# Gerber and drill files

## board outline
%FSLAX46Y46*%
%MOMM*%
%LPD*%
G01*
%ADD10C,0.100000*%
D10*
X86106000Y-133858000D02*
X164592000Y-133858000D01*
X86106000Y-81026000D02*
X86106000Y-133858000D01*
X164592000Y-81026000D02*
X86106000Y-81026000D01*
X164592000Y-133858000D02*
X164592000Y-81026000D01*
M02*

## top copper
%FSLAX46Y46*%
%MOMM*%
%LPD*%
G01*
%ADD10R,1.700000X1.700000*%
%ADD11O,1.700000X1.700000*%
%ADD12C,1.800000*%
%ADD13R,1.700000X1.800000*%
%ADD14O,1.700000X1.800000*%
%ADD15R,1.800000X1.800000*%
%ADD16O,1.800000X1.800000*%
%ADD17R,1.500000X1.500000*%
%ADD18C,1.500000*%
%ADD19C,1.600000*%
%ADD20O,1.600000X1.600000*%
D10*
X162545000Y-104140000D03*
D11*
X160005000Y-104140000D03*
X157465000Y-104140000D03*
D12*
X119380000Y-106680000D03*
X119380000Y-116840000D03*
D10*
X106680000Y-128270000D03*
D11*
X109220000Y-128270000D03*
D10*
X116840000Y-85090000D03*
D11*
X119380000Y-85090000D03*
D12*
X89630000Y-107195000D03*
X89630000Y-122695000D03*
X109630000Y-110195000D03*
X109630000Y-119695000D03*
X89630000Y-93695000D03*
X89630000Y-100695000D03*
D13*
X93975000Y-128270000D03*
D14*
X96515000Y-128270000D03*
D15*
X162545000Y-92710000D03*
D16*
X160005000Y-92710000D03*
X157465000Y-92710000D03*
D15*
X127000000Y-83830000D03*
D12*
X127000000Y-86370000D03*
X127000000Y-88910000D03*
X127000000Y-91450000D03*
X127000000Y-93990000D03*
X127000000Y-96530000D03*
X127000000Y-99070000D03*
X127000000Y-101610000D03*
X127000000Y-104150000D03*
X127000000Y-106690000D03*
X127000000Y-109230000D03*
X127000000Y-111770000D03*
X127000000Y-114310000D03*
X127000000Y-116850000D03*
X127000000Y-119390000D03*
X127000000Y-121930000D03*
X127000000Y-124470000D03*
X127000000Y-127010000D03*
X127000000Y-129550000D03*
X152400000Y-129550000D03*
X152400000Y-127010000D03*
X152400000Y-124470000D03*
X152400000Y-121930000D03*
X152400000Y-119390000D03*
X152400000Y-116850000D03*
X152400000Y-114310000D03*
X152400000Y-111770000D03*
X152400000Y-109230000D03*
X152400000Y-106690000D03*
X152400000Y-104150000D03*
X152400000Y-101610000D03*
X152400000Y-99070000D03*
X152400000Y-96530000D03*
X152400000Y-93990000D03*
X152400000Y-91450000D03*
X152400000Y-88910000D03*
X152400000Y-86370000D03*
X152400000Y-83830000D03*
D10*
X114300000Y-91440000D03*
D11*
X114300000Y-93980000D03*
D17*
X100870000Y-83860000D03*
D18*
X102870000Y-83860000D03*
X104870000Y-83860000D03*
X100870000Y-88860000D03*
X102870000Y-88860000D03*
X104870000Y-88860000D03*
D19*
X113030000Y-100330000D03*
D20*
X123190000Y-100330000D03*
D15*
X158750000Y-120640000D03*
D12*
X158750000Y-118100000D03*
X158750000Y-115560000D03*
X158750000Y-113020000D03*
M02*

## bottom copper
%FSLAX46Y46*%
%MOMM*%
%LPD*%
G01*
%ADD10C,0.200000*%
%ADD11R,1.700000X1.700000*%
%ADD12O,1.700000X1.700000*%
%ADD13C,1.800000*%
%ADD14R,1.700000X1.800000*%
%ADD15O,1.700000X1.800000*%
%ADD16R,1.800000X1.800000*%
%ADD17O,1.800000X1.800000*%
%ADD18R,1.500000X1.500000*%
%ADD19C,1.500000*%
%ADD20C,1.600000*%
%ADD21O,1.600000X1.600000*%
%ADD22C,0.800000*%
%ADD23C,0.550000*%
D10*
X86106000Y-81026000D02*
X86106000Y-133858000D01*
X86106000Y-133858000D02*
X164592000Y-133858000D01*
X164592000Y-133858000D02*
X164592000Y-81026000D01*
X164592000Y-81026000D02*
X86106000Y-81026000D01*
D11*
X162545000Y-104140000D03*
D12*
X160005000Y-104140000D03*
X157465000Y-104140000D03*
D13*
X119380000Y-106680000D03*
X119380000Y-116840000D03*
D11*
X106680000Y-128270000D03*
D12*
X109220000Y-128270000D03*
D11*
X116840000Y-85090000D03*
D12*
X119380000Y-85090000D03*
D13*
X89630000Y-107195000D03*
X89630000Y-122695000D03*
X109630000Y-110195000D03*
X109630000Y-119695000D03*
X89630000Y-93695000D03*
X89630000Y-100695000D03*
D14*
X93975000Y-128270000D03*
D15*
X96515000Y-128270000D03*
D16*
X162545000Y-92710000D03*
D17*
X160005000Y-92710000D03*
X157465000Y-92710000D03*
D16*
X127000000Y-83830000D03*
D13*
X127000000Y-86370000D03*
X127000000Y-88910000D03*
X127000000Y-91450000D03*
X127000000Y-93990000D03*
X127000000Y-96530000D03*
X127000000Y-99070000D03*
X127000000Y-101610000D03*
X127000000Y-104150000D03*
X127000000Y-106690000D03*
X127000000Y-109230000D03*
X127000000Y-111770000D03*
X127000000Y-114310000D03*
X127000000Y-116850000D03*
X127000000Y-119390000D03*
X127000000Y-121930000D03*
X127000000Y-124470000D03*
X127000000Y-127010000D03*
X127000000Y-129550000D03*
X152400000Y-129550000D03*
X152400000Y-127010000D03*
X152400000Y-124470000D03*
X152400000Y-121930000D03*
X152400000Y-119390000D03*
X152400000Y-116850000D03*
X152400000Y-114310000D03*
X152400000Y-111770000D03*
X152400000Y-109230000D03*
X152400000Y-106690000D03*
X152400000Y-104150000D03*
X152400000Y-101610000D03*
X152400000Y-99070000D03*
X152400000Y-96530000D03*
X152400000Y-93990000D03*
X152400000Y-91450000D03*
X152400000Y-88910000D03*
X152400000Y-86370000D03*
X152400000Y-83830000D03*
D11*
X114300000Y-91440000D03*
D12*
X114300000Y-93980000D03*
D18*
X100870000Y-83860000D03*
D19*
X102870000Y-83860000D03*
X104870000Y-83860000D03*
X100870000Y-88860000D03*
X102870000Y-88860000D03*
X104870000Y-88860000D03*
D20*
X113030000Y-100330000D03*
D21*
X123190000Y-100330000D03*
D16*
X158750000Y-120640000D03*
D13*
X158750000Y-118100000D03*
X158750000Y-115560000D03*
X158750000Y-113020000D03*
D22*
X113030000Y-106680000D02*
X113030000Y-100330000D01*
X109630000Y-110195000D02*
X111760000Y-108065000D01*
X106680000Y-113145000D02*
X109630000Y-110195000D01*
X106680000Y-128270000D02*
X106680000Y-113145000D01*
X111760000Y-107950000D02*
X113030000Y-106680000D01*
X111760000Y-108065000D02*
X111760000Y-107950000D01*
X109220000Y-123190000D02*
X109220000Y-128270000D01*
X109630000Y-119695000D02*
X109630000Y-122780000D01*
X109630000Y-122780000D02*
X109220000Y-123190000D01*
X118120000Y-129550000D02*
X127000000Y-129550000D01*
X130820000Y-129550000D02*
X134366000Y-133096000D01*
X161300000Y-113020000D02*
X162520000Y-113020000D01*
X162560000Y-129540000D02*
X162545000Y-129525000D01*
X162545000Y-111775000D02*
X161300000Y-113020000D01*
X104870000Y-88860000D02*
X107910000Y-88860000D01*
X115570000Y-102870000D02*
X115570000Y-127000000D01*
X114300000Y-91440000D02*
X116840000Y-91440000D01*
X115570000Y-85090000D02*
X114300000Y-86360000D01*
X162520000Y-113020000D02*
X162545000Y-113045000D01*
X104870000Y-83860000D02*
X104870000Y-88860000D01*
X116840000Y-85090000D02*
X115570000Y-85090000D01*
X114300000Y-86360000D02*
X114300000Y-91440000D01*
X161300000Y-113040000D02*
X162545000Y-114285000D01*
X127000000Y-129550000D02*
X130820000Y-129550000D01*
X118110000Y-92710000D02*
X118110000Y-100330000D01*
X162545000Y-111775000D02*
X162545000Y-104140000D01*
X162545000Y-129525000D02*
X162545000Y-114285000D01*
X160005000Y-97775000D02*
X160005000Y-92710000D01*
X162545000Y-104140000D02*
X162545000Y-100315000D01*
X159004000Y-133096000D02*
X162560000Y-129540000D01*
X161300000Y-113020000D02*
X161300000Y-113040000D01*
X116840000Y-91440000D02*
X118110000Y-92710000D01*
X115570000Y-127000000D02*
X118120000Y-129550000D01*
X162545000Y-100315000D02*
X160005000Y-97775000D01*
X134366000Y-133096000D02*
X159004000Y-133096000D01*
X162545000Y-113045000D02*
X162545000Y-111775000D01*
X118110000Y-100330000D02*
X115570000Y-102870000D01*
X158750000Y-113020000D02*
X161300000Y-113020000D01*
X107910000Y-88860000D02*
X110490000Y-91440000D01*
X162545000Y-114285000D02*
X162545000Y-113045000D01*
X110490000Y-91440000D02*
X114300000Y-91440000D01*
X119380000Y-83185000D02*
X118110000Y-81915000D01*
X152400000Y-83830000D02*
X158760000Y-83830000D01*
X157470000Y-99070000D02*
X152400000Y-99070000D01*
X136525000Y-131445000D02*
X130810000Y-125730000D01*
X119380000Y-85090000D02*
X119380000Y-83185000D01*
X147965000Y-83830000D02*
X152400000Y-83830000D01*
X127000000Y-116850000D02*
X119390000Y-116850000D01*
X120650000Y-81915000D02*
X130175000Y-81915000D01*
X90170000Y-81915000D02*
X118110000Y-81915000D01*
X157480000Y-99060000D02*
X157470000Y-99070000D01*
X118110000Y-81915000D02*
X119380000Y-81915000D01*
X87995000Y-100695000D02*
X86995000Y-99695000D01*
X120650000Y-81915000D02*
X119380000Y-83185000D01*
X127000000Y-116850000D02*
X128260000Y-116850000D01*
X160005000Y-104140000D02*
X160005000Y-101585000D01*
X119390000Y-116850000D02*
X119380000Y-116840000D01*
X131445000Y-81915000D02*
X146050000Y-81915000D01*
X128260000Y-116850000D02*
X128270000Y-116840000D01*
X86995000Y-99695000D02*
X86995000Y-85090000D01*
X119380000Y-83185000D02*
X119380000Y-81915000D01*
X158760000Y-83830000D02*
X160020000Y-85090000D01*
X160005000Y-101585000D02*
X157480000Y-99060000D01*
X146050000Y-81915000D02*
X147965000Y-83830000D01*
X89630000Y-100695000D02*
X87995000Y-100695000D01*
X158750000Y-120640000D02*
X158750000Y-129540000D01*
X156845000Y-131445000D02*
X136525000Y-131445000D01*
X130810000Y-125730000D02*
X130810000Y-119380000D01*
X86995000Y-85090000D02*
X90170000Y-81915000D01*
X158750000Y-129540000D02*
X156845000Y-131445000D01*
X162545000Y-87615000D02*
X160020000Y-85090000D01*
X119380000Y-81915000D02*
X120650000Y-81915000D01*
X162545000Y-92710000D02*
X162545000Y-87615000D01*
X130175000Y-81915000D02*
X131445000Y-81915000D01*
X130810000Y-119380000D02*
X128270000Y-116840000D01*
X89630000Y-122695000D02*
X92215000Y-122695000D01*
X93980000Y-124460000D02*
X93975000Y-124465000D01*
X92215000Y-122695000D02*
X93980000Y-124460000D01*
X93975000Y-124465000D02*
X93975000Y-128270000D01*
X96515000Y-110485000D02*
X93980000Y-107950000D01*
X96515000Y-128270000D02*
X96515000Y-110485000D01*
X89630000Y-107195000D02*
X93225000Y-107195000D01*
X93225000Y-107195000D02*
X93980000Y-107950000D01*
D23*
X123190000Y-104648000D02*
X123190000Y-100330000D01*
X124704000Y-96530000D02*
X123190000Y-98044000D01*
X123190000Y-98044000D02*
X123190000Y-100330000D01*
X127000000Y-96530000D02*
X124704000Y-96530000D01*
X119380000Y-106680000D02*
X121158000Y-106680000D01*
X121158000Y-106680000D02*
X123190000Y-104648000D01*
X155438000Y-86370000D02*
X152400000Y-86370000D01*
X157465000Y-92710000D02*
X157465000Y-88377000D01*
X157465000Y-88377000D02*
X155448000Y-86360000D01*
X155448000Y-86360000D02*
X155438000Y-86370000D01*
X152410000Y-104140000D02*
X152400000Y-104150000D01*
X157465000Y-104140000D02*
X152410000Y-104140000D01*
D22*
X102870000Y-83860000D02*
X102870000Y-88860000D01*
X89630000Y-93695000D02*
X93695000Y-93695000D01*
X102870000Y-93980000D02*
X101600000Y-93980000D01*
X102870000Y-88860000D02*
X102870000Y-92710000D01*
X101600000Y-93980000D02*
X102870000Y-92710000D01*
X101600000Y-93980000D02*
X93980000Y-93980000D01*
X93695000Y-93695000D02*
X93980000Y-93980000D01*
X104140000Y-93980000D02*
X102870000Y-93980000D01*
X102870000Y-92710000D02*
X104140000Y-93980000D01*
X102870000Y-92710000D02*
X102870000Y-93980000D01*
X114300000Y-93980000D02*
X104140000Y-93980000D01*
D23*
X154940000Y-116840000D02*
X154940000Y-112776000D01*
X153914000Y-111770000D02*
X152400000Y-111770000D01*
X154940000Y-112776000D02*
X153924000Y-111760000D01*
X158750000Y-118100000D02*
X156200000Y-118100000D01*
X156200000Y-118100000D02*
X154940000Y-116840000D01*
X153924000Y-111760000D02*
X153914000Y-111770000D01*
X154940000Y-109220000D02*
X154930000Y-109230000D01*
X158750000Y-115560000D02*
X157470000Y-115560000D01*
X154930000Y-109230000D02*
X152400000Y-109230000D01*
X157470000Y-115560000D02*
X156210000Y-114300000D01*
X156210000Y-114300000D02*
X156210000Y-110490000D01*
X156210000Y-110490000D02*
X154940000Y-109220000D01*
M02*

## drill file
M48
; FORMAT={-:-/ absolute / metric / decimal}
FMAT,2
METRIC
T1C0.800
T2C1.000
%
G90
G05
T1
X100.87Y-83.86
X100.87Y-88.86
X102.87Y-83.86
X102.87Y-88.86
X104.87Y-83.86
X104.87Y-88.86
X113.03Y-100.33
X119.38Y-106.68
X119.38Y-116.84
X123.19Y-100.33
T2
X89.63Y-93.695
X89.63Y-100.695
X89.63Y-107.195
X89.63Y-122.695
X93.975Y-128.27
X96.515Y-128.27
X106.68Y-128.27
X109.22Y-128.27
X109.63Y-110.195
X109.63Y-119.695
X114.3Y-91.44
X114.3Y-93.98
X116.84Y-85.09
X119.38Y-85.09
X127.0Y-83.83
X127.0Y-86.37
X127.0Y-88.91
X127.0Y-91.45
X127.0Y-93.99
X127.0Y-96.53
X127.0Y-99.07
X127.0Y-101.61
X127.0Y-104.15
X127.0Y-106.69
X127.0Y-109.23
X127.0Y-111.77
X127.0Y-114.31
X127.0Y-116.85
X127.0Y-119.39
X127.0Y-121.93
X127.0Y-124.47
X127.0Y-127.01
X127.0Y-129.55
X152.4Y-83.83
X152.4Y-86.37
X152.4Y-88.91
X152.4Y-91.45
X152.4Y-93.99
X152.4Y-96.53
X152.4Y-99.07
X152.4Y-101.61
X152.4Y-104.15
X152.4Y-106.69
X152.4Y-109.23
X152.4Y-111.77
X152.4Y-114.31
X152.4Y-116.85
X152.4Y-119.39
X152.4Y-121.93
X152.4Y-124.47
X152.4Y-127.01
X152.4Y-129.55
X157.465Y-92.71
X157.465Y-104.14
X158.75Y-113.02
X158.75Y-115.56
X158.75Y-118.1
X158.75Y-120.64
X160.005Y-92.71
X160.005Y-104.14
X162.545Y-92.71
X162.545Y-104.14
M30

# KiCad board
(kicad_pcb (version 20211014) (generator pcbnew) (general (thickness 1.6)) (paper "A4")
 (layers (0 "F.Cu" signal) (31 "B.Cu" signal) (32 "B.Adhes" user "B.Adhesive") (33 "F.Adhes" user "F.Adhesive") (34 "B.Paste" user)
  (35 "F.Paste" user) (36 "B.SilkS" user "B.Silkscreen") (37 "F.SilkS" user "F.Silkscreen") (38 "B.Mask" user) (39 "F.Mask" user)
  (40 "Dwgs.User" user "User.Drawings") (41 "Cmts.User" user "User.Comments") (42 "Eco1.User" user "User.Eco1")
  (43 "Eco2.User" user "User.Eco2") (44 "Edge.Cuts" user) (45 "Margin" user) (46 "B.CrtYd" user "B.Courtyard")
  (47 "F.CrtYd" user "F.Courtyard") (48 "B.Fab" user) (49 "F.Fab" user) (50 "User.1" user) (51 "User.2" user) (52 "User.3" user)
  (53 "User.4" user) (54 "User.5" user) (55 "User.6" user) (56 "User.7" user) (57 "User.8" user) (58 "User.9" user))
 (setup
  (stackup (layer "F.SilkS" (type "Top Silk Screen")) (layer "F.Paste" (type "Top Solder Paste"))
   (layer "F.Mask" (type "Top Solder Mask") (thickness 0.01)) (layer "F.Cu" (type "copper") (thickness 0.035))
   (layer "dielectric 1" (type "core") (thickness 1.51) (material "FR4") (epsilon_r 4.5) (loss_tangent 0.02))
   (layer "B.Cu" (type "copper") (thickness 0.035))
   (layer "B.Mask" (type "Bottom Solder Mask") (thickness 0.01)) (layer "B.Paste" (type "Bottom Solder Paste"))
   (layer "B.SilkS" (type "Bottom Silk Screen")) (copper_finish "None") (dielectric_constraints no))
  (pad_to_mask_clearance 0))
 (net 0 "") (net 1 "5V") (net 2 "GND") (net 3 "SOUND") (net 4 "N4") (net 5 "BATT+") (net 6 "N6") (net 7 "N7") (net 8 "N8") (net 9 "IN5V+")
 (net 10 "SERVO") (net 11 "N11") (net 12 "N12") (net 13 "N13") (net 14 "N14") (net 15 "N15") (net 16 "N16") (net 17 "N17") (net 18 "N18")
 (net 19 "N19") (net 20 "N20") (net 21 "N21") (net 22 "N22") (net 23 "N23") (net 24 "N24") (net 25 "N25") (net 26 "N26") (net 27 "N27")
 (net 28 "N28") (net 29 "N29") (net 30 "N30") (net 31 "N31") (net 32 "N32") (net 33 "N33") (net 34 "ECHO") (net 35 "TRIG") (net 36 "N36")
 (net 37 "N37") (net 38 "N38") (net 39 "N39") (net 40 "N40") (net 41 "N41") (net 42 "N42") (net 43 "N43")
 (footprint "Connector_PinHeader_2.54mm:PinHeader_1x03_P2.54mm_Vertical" (layer "F.Cu") (at 162.545 104.14 -90)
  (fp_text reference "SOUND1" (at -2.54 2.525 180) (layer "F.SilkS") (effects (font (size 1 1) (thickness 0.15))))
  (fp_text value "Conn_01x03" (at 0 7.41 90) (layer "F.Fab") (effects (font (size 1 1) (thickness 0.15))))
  (pad "1" thru_hole rect (at 0 0 270) (size 1.7 1.7) (drill 1) (layers *.Cu *.Mask) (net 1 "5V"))
  (pad "2" thru_hole oval (at 0 2.54 270) (size 1.7 1.7) (drill 1) (layers *.Cu *.Mask) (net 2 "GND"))
  (pad "3" thru_hole oval (at 0 5.08 270) (size 1.7 1.7) (drill 1) (layers *.Cu *.Mask) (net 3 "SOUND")))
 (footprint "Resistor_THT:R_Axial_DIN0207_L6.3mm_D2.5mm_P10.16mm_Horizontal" (layer "F.Cu") (at 119.38 106.68 -90)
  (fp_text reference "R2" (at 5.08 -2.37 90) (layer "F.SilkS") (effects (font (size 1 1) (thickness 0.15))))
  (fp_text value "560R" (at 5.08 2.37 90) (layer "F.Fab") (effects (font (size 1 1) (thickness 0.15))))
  (pad "1" thru_hole circle (at 0 0 270) (size 1.8 1.8) (drill 0.8) (layers *.Cu *.Mask) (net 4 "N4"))
  (pad "2" thru_hole circle (at 10.16 0 270) (size 1.8 1.8) (drill 0.8) (layers *.Cu *.Mask) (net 2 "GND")))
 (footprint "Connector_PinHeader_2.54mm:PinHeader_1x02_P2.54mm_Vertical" (layer "F.Cu") (at 106.68 128.27 90)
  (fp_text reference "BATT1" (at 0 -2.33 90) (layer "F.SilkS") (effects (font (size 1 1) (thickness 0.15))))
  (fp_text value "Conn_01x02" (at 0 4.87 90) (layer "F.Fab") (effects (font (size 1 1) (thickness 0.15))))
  (pad "1" thru_hole rect (at 0 0 90) (size 1.7 1.7) (drill 1) (layers *.Cu *.Mask) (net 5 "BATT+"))
  (pad "2" thru_hole oval (at 0 2.54 90) (size 1.7 1.7) (drill 1) (layers *.Cu *.Mask) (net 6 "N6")))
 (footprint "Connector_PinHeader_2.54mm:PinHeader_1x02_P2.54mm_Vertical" (layer "F.Cu") (at 116.84 85.09 90)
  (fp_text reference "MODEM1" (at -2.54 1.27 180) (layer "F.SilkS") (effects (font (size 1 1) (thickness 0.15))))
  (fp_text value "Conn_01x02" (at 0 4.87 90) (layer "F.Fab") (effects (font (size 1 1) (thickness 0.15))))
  (pad "1" thru_hole rect (at 0 0 90) (size 1.7 1.7) (drill 1) (layers *.Cu *.Mask) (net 1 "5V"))
  (pad "2" thru_hole oval (at 0 2.54 90) (size 1.7 1.7) (drill 1) (layers *.Cu *.Mask) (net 2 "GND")))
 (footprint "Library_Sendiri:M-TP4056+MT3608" (layer "F.Cu") (at 102.87 107.315 90)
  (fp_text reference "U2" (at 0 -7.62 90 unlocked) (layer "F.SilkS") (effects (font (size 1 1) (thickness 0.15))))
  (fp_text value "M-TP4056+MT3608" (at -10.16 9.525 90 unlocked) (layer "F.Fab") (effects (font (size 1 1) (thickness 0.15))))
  (pad "1" thru_hole circle (at 0.12 -13.24 90) (size 1.8 1.8) (drill 1) (layers *.Cu *.Mask) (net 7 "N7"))
  (pad "2" thru_hole circle (at -15.38 -13.24 90) (size 1.8 1.8) (drill 1) (layers *.Cu *.Mask) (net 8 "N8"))
  (pad "3" thru_hole circle (at -2.88 6.76 90) (size 1.8 1.8) (drill 1) (layers *.Cu *.Mask) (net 5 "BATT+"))
  (pad "4" thru_hole circle (at -12.38 6.76 90) (size 1.8 1.8) (drill 1) (layers *.Cu *.Mask) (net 6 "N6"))
  (pad "5" thru_hole circle (at 13.62 -13.24 90) (size 1.8 1.8) (drill 1) (layers *.Cu *.Mask) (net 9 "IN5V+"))
  (pad "6" thru_hole circle (at 6.62 -13.24 90) (size 1.8 1.8) (drill 1) (layers *.Cu *.Mask) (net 2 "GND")))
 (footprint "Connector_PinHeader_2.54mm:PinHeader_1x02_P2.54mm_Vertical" (layer "F.Cu") (at 93.975 128.27 90)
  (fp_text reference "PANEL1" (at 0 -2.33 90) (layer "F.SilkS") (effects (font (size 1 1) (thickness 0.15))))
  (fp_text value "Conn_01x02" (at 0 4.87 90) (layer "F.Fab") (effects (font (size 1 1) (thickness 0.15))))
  (pad "1" thru_hole rect (at 0 0 90) (size 1.8 1.7) (drill 1) (layers *.Cu *.Mask) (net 8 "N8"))
  (pad "2" thru_hole oval (at 0 2.54 90) (size 1.8 1.7) (drill 1) (layers *.Cu *.Mask) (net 7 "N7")))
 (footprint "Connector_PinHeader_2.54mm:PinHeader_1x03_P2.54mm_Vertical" (layer "F.Cu") (at 162.545 92.71 -90)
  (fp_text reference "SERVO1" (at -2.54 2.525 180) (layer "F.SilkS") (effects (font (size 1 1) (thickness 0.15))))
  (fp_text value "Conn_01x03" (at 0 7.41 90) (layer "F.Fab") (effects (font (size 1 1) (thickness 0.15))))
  (pad "1" thru_hole rect (at 0 0 270) (size 1.8 1.8) (drill 1) (layers *.Cu *.Mask) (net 2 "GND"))
  (pad "2" thru_hole oval (at 0 2.54 270) (size 1.8 1.8) (drill 1) (layers *.Cu *.Mask) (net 1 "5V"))
  (pad "3" thru_hole oval (at 0 5.08 270) (size 1.8 1.8) (drill 1) (layers *.Cu *.Mask) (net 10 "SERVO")))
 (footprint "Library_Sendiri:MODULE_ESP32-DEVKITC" (layer "F.Cu") (at 139.7 106.68)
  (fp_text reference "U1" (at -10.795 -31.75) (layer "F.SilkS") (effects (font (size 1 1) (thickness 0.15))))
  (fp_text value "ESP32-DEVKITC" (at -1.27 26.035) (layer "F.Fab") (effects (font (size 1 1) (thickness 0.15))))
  (pad "1" thru_hole rect (at -12.7 -22.85) (size 1.8 1.8) (drill 1) (layers *.Cu *.Mask) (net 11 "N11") (solder_mask_margin 0.102))
  (pad "2" thru_hole circle (at -12.7 -20.31) (size 1.8 1.8) (drill 1) (layers *.Cu *.Mask) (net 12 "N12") (solder_mask_margin 0.102))
  (pad "3" thru_hole circle (at -12.7 -17.77) (size 1.8 1.8) (drill 1) (layers *.Cu *.Mask) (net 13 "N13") (solder_mask_margin 0.102))
  (pad "4" thru_hole circle (at -12.7 -15.23) (size 1.8 1.8) (drill 1) (layers *.Cu *.Mask) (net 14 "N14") (solder_mask_margin 0.102))
  (pad "5" thru_hole circle (at -12.7 -12.69) (size 1.8 1.8) (drill 1) (layers *.Cu *.Mask) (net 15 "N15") (solder_mask_margin 0.102))
  (pad "6" thru_hole circle (at -12.7 -10.15) (size 1.8 1.8) (drill 1) (layers *.Cu *.Mask) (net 4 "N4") (solder_mask_margin 0.102))
  (pad "7" thru_hole circle (at -12.7 -7.61) (size 1.8 1.8) (drill 1) (layers *.Cu *.Mask) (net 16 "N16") (solder_mask_margin 0.102))
  (pad "8" thru_hole circle (at -12.7 -5.07) (size 1.8 1.8) (drill 1) (layers *.Cu *.Mask) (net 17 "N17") (solder_mask_margin 0.102))
  (pad "9" thru_hole circle (at -12.7 -2.53) (size 1.8 1.8) (drill 1) (layers *.Cu *.Mask) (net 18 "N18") (solder_mask_margin 0.102))
  (pad "10" thru_hole circle (at -12.7 0.01) (size 1.8 1.8) (drill 1) (layers *.Cu *.Mask) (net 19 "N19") (solder_mask_margin 0.102))
  (pad "11" thru_hole circle (at -12.7 2.55) (size 1.8 1.8) (drill 1) (layers *.Cu *.Mask) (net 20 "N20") (solder_mask_margin 0.102))
  (pad "12" thru_hole circle (at -12.7 5.09) (size 1.8 1.8) (drill 1) (layers *.Cu *.Mask) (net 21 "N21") (solder_mask_margin 0.102))
  (pad "13" thru_hole circle (at -12.7 7.63) (size 1.8 1.8) (drill 1) (layers *.Cu *.Mask) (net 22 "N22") (solder_mask_margin 0.102))
  (pad "14" thru_hole circle (at -12.7 10.17) (size 1.8 1.8) (drill 1) (layers *.Cu *.Mask) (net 2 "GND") (solder_mask_margin 0.102))
  (pad "15" thru_hole circle (at -12.7 12.71) (size 1.8 1.8) (drill 1) (layers *.Cu *.Mask) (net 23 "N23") (solder_mask_margin 0.102))
  (pad "16" thru_hole circle (at -12.7 15.25) (size 1.8 1.8) (drill 1) (layers *.Cu *.Mask) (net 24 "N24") (solder_mask_margin 0.102))
  (pad "17" thru_hole circle (at -12.7 17.79) (size 1.8 1.8) (drill 1) (layers *.Cu *.Mask) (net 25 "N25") (solder_mask_margin 0.102))
  (pad "18" thru_hole circle (at -12.7 20.33) (size 1.8 1.8) (drill 1) (layers *.Cu *.Mask) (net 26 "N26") (solder_mask_margin 0.102))
  (pad "19" thru_hole circle (at -12.7 22.87) (size 1.8 1.8) (drill 1) (layers *.Cu *.Mask) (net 1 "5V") (solder_mask_margin 0.102))
  (pad "20" thru_hole circle (at 12.7 22.87) (size 1.8 1.8) (drill 1) (layers *.Cu *.Mask) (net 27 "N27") (solder_mask_margin 0.102))
  (pad "21" thru_hole circle (at 12.7 20.33) (size 1.8 1.8) (drill 1) (layers *.Cu *.Mask) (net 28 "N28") (solder_mask_margin 0.102))
  (pad "22" thru_hole circle (at 12.7 17.79) (size 1.8 1.8) (drill 1) (layers *.Cu *.Mask) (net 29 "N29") (solder_mask_margin 0.102))
  (pad "23" thru_hole circle (at 12.7 15.25) (size 1.8 1.8) (drill 1) (layers *.Cu *.Mask) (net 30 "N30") (solder_mask_margin 0.102))
  (pad "24" thru_hole circle (at 12.7 12.71) (size 1.8 1.8) (drill 1) (layers *.Cu *.Mask) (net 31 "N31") (solder_mask_margin 0.102))
  (pad "25" thru_hole circle (at 12.7 10.17) (size 1.8 1.8) (drill 1) (layers *.Cu *.Mask) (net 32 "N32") (solder_mask_margin 0.102))
  (pad "26" thru_hole circle (at 12.7 7.63) (size 1.8 1.8) (drill 1) (layers *.Cu *.Mask) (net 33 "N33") (solder_mask_margin 0.102))
  (pad "27" thru_hole circle (at 12.7 5.09) (size 1.8 1.8) (drill 1) (layers *.Cu *.Mask) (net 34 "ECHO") (solder_mask_margin 0.102))
  (pad "28" thru_hole circle (at 12.7 2.55) (size 1.8 1.8) (drill 1) (layers *.Cu *.Mask) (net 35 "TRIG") (solder_mask_margin 0.102))
  (pad "29" thru_hole circle (at 12.7 0.01) (size 1.8 1.8) (drill 1) (layers *.Cu *.Mask) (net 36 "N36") (solder_mask_margin 0.102))
  (pad "30" thru_hole circle (at 12.7 -2.53) (size 1.8 1.8) (drill 1) (layers *.Cu *.Mask) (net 3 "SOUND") (solder_mask_margin 0.102))
  (pad "31" thru_hole circle (at 12.7 -5.07) (size 1.8 1.8) (drill 1) (layers *.Cu *.Mask) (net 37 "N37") (solder_mask_margin 0.102))
  (pad "32" thru_hole circle (at 12.7 -7.61) (size 1.8 1.8) (drill 1) (layers *.Cu *.Mask) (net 2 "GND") (solder_mask_margin 0.102))
  (pad "33" thru_hole circle (at 12.7 -10.15) (size 1.8 1.8) (drill 1) (layers *.Cu *.Mask) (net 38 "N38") (solder_mask_margin 0.102))
  (pad "34" thru_hole circle (at 12.7 -12.69) (size 1.8 1.8) (drill 1) (layers *.Cu *.Mask) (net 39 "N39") (solder_mask_margin 0.102))
  (pad "35" thru_hole circle (at 12.7 -15.23) (size 1.8 1.8) (drill 1) (layers *.Cu *.Mask) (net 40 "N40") (solder_mask_margin 0.102))
  (pad "36" thru_hole circle (at 12.7 -17.77) (size 1.8 1.8) (drill 1) (layers *.Cu *.Mask) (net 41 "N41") (solder_mask_margin 0.102))
  (pad "37" thru_hole circle (at 12.7 -20.31) (size 1.8 1.8) (drill 1) (layers *.Cu *.Mask) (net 10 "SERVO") (solder_mask_margin 0.102))
  (pad "38" thru_hole circle (at 12.7 -22.85) (size 1.8 1.8) (drill 1) (layers *.Cu *.Mask) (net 2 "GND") (solder_mask_margin 0.102)))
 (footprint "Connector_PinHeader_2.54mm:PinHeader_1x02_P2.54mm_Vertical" (layer "F.Cu") (at 114.3 91.44)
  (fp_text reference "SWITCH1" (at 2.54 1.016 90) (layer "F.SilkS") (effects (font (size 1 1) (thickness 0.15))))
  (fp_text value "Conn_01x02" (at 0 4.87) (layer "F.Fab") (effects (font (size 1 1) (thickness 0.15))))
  (pad "1" thru_hole rect (at 0 0) (size 1.7 1.7) (drill 1) (layers *.Cu *.Mask) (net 1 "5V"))
  (pad "2" thru_hole oval (at 0 2.54) (size 1.7 1.7) (drill 1) (layers *.Cu *.Mask) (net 9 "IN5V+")))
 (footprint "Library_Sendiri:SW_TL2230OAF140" (layer "F.Cu") (at 102.87 86.36)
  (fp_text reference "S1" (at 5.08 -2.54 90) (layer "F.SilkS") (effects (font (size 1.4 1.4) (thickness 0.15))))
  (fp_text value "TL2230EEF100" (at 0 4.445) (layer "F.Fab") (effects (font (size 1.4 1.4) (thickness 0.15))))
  (pad "1" thru_hole rect (at -2 -2.5) (size 1.5 1.5) (drill 0.8) (layers *.Cu *.Mask) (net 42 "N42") (solder_mask_margin 0.102))
  (pad "2" thru_hole circle (at 0 -2.5) (size 1.5 1.5) (drill 0.8) (layers *.Cu *.Mask) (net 9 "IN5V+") (solder_mask_margin 0.102))
  (pad "3" thru_hole circle (at 2 -2.5) (size 1.5 1.5) (drill 0.8) (layers *.Cu *.Mask) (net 1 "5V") (solder_mask_margin 0.102))
  (pad "4" thru_hole circle (at -2 2.5) (size 1.5 1.5) (drill 0.8) (layers *.Cu *.Mask) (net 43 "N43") (solder_mask_margin 0.102))
  (pad "5" thru_hole circle (at 0 2.5) (size 1.5 1.5) (drill 0.8) (layers *.Cu *.Mask) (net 9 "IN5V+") (solder_mask_margin 0.102))
  (pad "6" thru_hole circle (at 2 2.5) (size 1.5 1.5) (drill 0.8) (layers *.Cu *.Mask) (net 1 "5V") (solder_mask_margin 0.102)))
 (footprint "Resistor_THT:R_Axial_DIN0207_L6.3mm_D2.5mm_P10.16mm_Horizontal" (layer "F.Cu") (at 113.03 100.33)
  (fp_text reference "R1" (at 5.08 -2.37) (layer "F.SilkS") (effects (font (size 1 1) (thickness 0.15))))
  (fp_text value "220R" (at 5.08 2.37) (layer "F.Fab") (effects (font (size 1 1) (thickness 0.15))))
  (pad "1" thru_hole circle (at 0 0) (size 1.6 1.6) (drill 0.8) (layers *.Cu *.Mask) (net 5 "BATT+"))
  (pad "2" thru_hole oval (at 10.16 0) (size 1.6 1.6) (drill 0.8) (layers *.Cu *.Mask) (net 4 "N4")))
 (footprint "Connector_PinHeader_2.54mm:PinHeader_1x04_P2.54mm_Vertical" (layer "F.Cu") (at 158.75 120.64 180)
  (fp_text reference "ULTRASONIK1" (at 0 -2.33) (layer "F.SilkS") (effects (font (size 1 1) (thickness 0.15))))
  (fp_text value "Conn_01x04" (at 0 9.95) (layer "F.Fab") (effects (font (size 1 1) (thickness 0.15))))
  (pad "1" thru_hole rect (at 0 0 180) (size 1.8 1.8) (drill 1) (layers *.Cu *.Mask) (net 2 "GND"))
  (pad "2" thru_hole circle (at 0 2.54 180) (size 1.8 1.8) (drill 1) (layers *.Cu *.Mask) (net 34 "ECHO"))
  (pad "3" thru_hole circle (at 0 5.08 180) (size 1.8 1.8) (drill 1) (layers *.Cu *.Mask) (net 35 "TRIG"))
  (pad "4" thru_hole circle (at 0 7.62 180) (size 1.8 1.8) (drill 1) (layers *.Cu *.Mask) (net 1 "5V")))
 (gr_line (start 86.106 81.026) (end 86.106 133.858) (layer "B.Cu") (width 0.2))
 (gr_line (start 86.106 133.858) (end 164.592 133.858) (layer "B.Cu") (width 0.2))
 (gr_line (start 164.592 133.858) (end 164.592 81.026) (layer "B.Cu") (width 0.2))
 (gr_line (start 164.592 81.026) (end 86.106 81.026) (layer "B.Cu") (width 0.2))
 (gr_line (start 86.106 133.858) (end 164.592 133.858) (layer "Edge.Cuts") (width 0.1))
 (gr_line (start 86.106 81.026) (end 86.106 133.858) (layer "Edge.Cuts") (width 0.1))
 (gr_line (start 164.592 81.026) (end 86.106 81.026) (layer "Edge.Cuts") (width 0.1))
 (gr_line (start 164.592 133.858) (end 164.592 81.026) (layer "Edge.Cuts") (width 0.1))
 (segment (start 113.03 106.68) (end 113.03 100.33) (width 0.8) (layer "B.Cu") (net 5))
 (segment (start 109.63 110.195) (end 111.76 108.065) (width 0.8) (layer "B.Cu") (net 5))
 (segment (start 106.68 113.145) (end 109.63 110.195) (width 0.8) (layer "B.Cu") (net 5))
 (segment (start 106.68 128.27) (end 106.68 113.145) (width 0.8) (layer "B.Cu") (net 5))
 (segment (start 111.76 107.95) (end 113.03 106.68) (width 0.8) (layer "B.Cu") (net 5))
 (segment (start 111.76 108.065) (end 111.76 107.95) (width 0.8) (layer "B.Cu") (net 5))
 (segment (start 109.22 123.19) (end 109.22 128.27) (width 0.8) (layer "B.Cu") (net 6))
 (segment (start 109.63 119.695) (end 109.63 122.78) (width 0.8) (layer "B.Cu") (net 6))
 (segment (start 109.63 122.78) (end 109.22 123.19) (width 0.8) (layer "B.Cu") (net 6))
 (segment (start 118.12 129.55) (end 127 129.55) (width 0.8) (layer "B.Cu") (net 1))
 (segment (start 130.82 129.55) (end 134.366 133.096) (width 0.8) (layer "B.Cu") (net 1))
 (segment (start 161.3 113.02) (end 162.52 113.02) (width 0.8) (layer "B.Cu") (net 1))
 (segment (start 162.56 129.54) (end 162.545 129.525) (width 0.8) (layer "B.Cu") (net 1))
 (segment (start 162.545 111.775) (end 161.3 113.02) (width 0.8) (layer "B.Cu") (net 1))
 (segment (start 104.87 88.86) (end 107.91 88.86) (width 0.8) (layer "B.Cu") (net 1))
 (segment (start 115.57 102.87) (end 115.57 127) (width 0.8) (layer "B.Cu") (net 1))
 (segment (start 114.3 91.44) (end 116.84 91.44) (width 0.8) (layer "B.Cu") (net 1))
 (segment (start 115.57 85.09) (end 114.3 86.36) (width 0.8) (layer "B.Cu") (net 1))
 (segment (start 162.52 113.02) (end 162.545 113.045) (width 0.8) (layer "B.Cu") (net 1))
 (segment (start 104.87 83.86) (end 104.87 88.86) (width 0.8) (layer "B.Cu") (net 1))
 (segment (start 116.84 85.09) (end 115.57 85.09) (width 0.8) (layer "B.Cu") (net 1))
 (segment (start 114.3 86.36) (end 114.3 91.44) (width 0.8) (layer "B.Cu") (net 1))
 (segment (start 161.3 113.04) (end 162.545 114.285) (width 0.8) (layer "B.Cu") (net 1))
 (segment (start 127 129.55) (end 130.82 129.55) (width 0.8) (layer "B.Cu") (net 1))
 (segment (start 118.11 92.71) (end 118.11 100.33) (width 0.8) (layer "B.Cu") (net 1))
 (segment (start 162.545 111.775) (end 162.545 104.14) (width 0.8) (layer "B.Cu") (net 1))
 (segment (start 162.545 129.525) (end 162.545 114.285) (width 0.8) (layer "B.Cu") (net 1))
 (segment (start 160.005 97.775) (end 160.005 92.71) (width 0.8) (layer "B.Cu") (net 1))
 (segment (start 162.545 104.14) (end 162.545 100.315) (width 0.8) (layer "B.Cu") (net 1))
 (segment (start 159.004 133.096) (end 162.56 129.54) (width 0.8) (layer "B.Cu") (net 1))
 (segment (start 161.3 113.02) (end 161.3 113.04) (width 0.8) (layer "B.Cu") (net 1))
 (segment (start 116.84 91.44) (end 118.11 92.71) (width 0.8) (layer "B.Cu") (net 1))
 (segment (start 115.57 127) (end 118.12 129.55) (width 0.8) (layer "B.Cu") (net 1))
 (segment (start 162.545 100.315) (end 160.005 97.775) (width 0.8) (layer "B.Cu") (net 1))
 (segment (start 134.366 133.096) (end 159.004 133.096) (width 0.8) (layer "B.Cu") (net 1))
 (segment (start 162.545 113.045) (end 162.545 111.775) (width 0.8) (layer "B.Cu") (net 1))
 (segment (start 118.11 100.33) (end 115.57 102.87) (width 0.8) (layer "B.Cu") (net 1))
 (segment (start 158.75 113.02) (end 161.3 113.02) (width 0.8) (layer "B.Cu") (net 1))
 (segment (start 107.91 88.86) (end 110.49 91.44) (width 0.8) (layer "B.Cu") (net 1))
 (segment (start 162.545 114.285) (end 162.545 113.045) (width 0.8) (layer "B.Cu") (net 1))
 (segment (start 110.49 91.44) (end 114.3 91.44) (width 0.8) (layer "B.Cu") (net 1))
 (segment (start 119.38 83.185) (end 118.11 81.915) (width 0.8) (layer "B.Cu") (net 2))
 (segment (start 152.4 83.83) (end 158.76 83.83) (width 0.8) (layer "B.Cu") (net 2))
 (segment (start 157.47 99.07) (end 152.4 99.07) (width 0.8) (layer "B.Cu") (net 2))
 (segment (start 136.525 131.445) (end 130.81 125.73) (width 0.8) (layer "B.Cu") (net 2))
 (segment (start 119.38 85.09) (end 119.38 83.185) (width 0.8) (layer "B.Cu") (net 2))
 (segment (start 147.965 83.83) (end 152.4 83.83) (width 0.8) (layer "B.Cu") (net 2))
 (segment (start 127 116.85) (end 119.39 116.85) (width 0.8) (layer "B.Cu") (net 2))
 (segment (start 120.65 81.915) (end 130.175 81.915) (width 0.8) (layer "B.Cu") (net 2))
 (segment (start 90.17 81.915) (end 118.11 81.915) (width 0.8) (layer "B.Cu") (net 2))
 (segment (start 157.48 99.06) (end 157.47 99.07) (width 0.8) (layer "B.Cu") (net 2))
 (segment (start 118.11 81.915) (end 119.38 81.915) (width 0.8) (layer "B.Cu") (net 2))
 (segment (start 87.995 100.695) (end 86.995 99.695) (width 0.8) (layer "B.Cu") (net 2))
 (segment (start 120.65 81.915) (end 119.38 83.185) (width 0.8) (layer "B.Cu") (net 2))
 (segment (start 127 116.85) (end 128.26 116.85) (width 0.8) (layer "B.Cu") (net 2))
 (segment (start 160.005 104.14) (end 160.005 101.585) (width 0.8) (layer "B.Cu") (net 2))
 (segment (start 119.39 116.85) (end 119.38 116.84) (width 0.8) (layer "B.Cu") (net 2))
 (segment (start 131.445 81.915) (end 146.05 81.915) (width 0.8) (layer "B.Cu") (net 2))
 (segment (start 128.26 116.85) (end 128.27 116.84) (width 0.8) (layer "B.Cu") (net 2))
 (segment (start 86.995 99.695) (end 86.995 85.09) (width 0.8) (layer "B.Cu") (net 2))
 (segment (start 119.38 83.185) (end 119.38 81.915) (width 0.8) (layer "B.Cu") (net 2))
 (segment (start 158.76 83.83) (end 160.02 85.09) (width 0.8) (layer "B.Cu") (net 2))
 (segment (start 160.005 101.585) (end 157.48 99.06) (width 0.8) (layer "B.Cu") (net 2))
 (segment (start 146.05 81.915) (end 147.965 83.83) (width 0.8) (layer "B.Cu") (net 2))
 (segment (start 89.63 100.695) (end 87.995 100.695) (width 0.8) (layer "B.Cu") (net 2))
 (segment (start 158.75 120.64) (end 158.75 129.54) (width 0.8) (layer "B.Cu") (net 2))
 (segment (start 156.845 131.445) (end 136.525 131.445) (width 0.8) (layer "B.Cu") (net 2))
 (segment (start 130.81 125.73) (end 130.81 119.38) (width 0.8) (layer "B.Cu") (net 2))
 (segment (start 86.995 85.09) (end 90.17 81.915) (width 0.8) (layer "B.Cu") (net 2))
 (segment (start 158.75 129.54) (end 156.845 131.445) (width 0.8) (layer "B.Cu") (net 2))
 (segment (start 162.545 87.615) (end 160.02 85.09) (width 0.8) (layer "B.Cu") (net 2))
 (segment (start 119.38 81.915) (end 120.65 81.915) (width 0.8) (layer "B.Cu") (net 2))
 (segment (start 162.545 92.71) (end 162.545 87.615) (width 0.8) (layer "B.Cu") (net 2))
 (segment (start 130.175 81.915) (end 131.445 81.915) (width 0.8) (layer "B.Cu") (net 2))
 (segment (start 130.81 119.38) (end 128.27 116.84) (width 0.8) (layer "B.Cu") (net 2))
 (segment (start 89.63 122.695) (end 92.215 122.695) (width 0.8) (layer "B.Cu") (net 8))
 (segment (start 93.98 124.46) (end 93.975 124.465) (width 0.8) (layer "B.Cu") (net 8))
 (segment (start 92.215 122.695) (end 93.98 124.46) (width 0.8) (layer "B.Cu") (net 8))
 (segment (start 93.975 124.465) (end 93.975 128.27) (width 0.8) (layer "B.Cu") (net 8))
 (segment (start 96.515 110.485) (end 93.98 107.95) (width 0.8) (layer "B.Cu") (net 7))
 (segment (start 96.515 128.27) (end 96.515 110.485) (width 0.8) (layer "B.Cu") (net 7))
 (segment (start 89.63 107.195) (end 93.225 107.195) (width 0.8) (layer "B.Cu") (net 7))
 (segment (start 93.225 107.195) (end 93.98 107.95) (width 0.8) (layer "B.Cu") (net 7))
 (segment (start 123.19 104.648) (end 123.19 100.33) (width 0.55) (layer "B.Cu") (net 4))
 (segment (start 124.704 96.53) (end 123.19 98.044) (width 0.55) (layer "B.Cu") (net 4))
 (segment (start 123.19 98.044) (end 123.19 100.33) (width 0.55) (layer "B.Cu") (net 4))
 (segment (start 127 96.53) (end 124.704 96.53) (width 0.55) (layer "B.Cu") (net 4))
 (segment (start 119.38 106.68) (end 121.158 106.68) (width 0.55) (layer "B.Cu") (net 4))
 (segment (start 121.158 106.68) (end 123.19 104.648) (width 0.55) (layer "B.Cu") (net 4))
 (segment (start 155.438 86.37) (end 152.4 86.37) (width 0.55) (layer "B.Cu") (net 10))
 (segment (start 157.465 92.71) (end 157.465 88.377) (width 0.55) (layer "B.Cu") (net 10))
 (segment (start 157.465 88.377) (end 155.448 86.36) (width 0.55) (layer "B.Cu") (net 10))
 (segment (start 155.448 86.36) (end 155.438 86.37) (width 0.55) (layer "B.Cu") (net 10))
 (segment (start 152.41 104.14) (end 152.4 104.15) (width 0.55) (layer "B.Cu") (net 3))
 (segment (start 157.465 104.14) (end 152.41 104.14) (width 0.55) (layer "B.Cu") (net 3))
 (segment (start 102.87 83.86) (end 102.87 88.86) (width 0.8) (layer "B.Cu") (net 9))
 (segment (start 89.63 93.695) (end 93.695 93.695) (width 0.8) (layer "B.Cu") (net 9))
 (segment (start 102.87 93.98) (end 101.6 93.98) (width 0.8) (layer "B.Cu") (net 9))
 (segment (start 102.87 88.86) (end 102.87 92.71) (width 0.8) (layer "B.Cu") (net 9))
 (segment (start 101.6 93.98) (end 102.87 92.71) (width 0.8) (layer "B.Cu") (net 9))
 (segment (start 101.6 93.98) (end 93.98 93.98) (width 0.8) (layer "B.Cu") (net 9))
 (segment (start 93.695 93.695) (end 93.98 93.98) (width 0.8) (layer "B.Cu") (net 9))
 (segment (start 104.14 93.98) (end 102.87 93.98) (width 0.8) (layer "B.Cu") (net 9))
 (segment (start 102.87 92.71) (end 104.14 93.98) (width 0.8) (layer "B.Cu") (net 9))
 (segment (start 102.87 92.71) (end 102.87 93.98) (width 0.8) (layer "B.Cu") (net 9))
 (segment (start 114.3 93.98) (end 104.14 93.98) (width 0.8) (layer "B.Cu") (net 9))
 (segment (start 154.94 116.84) (end 154.94 112.776) (width 0.55) (layer "B.Cu") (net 34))
 (segment (start 153.914 111.77) (end 152.4 111.77) (width 0.55) (layer "B.Cu") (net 34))
 (segment (start 154.94 112.776) (end 153.924 111.76) (width 0.55) (layer "B.Cu") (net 34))
 (segment (start 158.75 118.1) (end 156.2 118.1) (width 0.55) (layer "B.Cu") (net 34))
 (segment (start 156.2 118.1) (end 154.94 116.84) (width 0.55) (layer "B.Cu") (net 34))
 (segment (start 153.924 111.76) (end 153.914 111.77) (width 0.55) (layer "B.Cu") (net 34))
 (segment (start 154.94 109.22) (end 154.93 109.23) (width 0.55) (layer "B.Cu") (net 35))
 (segment (start 158.75 115.56) (end 157.47 115.56) (width 0.55) (layer "B.Cu") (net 35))
 (segment (start 154.93 109.23) (end 152.4 109.23) (width 0.55) (layer "B.Cu") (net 35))
 (segment (start 157.47 115.56) (end 156.21 114.3) (width 0.55) (layer "B.Cu") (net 35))
 (segment (start 156.21 114.3) (end 156.21 110.49) (width 0.55) (layer "B.Cu") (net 35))
 (segment (start 156.21 110.49) (end 154.94 109.22) (width 0.55) (layer "B.Cu") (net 35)))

